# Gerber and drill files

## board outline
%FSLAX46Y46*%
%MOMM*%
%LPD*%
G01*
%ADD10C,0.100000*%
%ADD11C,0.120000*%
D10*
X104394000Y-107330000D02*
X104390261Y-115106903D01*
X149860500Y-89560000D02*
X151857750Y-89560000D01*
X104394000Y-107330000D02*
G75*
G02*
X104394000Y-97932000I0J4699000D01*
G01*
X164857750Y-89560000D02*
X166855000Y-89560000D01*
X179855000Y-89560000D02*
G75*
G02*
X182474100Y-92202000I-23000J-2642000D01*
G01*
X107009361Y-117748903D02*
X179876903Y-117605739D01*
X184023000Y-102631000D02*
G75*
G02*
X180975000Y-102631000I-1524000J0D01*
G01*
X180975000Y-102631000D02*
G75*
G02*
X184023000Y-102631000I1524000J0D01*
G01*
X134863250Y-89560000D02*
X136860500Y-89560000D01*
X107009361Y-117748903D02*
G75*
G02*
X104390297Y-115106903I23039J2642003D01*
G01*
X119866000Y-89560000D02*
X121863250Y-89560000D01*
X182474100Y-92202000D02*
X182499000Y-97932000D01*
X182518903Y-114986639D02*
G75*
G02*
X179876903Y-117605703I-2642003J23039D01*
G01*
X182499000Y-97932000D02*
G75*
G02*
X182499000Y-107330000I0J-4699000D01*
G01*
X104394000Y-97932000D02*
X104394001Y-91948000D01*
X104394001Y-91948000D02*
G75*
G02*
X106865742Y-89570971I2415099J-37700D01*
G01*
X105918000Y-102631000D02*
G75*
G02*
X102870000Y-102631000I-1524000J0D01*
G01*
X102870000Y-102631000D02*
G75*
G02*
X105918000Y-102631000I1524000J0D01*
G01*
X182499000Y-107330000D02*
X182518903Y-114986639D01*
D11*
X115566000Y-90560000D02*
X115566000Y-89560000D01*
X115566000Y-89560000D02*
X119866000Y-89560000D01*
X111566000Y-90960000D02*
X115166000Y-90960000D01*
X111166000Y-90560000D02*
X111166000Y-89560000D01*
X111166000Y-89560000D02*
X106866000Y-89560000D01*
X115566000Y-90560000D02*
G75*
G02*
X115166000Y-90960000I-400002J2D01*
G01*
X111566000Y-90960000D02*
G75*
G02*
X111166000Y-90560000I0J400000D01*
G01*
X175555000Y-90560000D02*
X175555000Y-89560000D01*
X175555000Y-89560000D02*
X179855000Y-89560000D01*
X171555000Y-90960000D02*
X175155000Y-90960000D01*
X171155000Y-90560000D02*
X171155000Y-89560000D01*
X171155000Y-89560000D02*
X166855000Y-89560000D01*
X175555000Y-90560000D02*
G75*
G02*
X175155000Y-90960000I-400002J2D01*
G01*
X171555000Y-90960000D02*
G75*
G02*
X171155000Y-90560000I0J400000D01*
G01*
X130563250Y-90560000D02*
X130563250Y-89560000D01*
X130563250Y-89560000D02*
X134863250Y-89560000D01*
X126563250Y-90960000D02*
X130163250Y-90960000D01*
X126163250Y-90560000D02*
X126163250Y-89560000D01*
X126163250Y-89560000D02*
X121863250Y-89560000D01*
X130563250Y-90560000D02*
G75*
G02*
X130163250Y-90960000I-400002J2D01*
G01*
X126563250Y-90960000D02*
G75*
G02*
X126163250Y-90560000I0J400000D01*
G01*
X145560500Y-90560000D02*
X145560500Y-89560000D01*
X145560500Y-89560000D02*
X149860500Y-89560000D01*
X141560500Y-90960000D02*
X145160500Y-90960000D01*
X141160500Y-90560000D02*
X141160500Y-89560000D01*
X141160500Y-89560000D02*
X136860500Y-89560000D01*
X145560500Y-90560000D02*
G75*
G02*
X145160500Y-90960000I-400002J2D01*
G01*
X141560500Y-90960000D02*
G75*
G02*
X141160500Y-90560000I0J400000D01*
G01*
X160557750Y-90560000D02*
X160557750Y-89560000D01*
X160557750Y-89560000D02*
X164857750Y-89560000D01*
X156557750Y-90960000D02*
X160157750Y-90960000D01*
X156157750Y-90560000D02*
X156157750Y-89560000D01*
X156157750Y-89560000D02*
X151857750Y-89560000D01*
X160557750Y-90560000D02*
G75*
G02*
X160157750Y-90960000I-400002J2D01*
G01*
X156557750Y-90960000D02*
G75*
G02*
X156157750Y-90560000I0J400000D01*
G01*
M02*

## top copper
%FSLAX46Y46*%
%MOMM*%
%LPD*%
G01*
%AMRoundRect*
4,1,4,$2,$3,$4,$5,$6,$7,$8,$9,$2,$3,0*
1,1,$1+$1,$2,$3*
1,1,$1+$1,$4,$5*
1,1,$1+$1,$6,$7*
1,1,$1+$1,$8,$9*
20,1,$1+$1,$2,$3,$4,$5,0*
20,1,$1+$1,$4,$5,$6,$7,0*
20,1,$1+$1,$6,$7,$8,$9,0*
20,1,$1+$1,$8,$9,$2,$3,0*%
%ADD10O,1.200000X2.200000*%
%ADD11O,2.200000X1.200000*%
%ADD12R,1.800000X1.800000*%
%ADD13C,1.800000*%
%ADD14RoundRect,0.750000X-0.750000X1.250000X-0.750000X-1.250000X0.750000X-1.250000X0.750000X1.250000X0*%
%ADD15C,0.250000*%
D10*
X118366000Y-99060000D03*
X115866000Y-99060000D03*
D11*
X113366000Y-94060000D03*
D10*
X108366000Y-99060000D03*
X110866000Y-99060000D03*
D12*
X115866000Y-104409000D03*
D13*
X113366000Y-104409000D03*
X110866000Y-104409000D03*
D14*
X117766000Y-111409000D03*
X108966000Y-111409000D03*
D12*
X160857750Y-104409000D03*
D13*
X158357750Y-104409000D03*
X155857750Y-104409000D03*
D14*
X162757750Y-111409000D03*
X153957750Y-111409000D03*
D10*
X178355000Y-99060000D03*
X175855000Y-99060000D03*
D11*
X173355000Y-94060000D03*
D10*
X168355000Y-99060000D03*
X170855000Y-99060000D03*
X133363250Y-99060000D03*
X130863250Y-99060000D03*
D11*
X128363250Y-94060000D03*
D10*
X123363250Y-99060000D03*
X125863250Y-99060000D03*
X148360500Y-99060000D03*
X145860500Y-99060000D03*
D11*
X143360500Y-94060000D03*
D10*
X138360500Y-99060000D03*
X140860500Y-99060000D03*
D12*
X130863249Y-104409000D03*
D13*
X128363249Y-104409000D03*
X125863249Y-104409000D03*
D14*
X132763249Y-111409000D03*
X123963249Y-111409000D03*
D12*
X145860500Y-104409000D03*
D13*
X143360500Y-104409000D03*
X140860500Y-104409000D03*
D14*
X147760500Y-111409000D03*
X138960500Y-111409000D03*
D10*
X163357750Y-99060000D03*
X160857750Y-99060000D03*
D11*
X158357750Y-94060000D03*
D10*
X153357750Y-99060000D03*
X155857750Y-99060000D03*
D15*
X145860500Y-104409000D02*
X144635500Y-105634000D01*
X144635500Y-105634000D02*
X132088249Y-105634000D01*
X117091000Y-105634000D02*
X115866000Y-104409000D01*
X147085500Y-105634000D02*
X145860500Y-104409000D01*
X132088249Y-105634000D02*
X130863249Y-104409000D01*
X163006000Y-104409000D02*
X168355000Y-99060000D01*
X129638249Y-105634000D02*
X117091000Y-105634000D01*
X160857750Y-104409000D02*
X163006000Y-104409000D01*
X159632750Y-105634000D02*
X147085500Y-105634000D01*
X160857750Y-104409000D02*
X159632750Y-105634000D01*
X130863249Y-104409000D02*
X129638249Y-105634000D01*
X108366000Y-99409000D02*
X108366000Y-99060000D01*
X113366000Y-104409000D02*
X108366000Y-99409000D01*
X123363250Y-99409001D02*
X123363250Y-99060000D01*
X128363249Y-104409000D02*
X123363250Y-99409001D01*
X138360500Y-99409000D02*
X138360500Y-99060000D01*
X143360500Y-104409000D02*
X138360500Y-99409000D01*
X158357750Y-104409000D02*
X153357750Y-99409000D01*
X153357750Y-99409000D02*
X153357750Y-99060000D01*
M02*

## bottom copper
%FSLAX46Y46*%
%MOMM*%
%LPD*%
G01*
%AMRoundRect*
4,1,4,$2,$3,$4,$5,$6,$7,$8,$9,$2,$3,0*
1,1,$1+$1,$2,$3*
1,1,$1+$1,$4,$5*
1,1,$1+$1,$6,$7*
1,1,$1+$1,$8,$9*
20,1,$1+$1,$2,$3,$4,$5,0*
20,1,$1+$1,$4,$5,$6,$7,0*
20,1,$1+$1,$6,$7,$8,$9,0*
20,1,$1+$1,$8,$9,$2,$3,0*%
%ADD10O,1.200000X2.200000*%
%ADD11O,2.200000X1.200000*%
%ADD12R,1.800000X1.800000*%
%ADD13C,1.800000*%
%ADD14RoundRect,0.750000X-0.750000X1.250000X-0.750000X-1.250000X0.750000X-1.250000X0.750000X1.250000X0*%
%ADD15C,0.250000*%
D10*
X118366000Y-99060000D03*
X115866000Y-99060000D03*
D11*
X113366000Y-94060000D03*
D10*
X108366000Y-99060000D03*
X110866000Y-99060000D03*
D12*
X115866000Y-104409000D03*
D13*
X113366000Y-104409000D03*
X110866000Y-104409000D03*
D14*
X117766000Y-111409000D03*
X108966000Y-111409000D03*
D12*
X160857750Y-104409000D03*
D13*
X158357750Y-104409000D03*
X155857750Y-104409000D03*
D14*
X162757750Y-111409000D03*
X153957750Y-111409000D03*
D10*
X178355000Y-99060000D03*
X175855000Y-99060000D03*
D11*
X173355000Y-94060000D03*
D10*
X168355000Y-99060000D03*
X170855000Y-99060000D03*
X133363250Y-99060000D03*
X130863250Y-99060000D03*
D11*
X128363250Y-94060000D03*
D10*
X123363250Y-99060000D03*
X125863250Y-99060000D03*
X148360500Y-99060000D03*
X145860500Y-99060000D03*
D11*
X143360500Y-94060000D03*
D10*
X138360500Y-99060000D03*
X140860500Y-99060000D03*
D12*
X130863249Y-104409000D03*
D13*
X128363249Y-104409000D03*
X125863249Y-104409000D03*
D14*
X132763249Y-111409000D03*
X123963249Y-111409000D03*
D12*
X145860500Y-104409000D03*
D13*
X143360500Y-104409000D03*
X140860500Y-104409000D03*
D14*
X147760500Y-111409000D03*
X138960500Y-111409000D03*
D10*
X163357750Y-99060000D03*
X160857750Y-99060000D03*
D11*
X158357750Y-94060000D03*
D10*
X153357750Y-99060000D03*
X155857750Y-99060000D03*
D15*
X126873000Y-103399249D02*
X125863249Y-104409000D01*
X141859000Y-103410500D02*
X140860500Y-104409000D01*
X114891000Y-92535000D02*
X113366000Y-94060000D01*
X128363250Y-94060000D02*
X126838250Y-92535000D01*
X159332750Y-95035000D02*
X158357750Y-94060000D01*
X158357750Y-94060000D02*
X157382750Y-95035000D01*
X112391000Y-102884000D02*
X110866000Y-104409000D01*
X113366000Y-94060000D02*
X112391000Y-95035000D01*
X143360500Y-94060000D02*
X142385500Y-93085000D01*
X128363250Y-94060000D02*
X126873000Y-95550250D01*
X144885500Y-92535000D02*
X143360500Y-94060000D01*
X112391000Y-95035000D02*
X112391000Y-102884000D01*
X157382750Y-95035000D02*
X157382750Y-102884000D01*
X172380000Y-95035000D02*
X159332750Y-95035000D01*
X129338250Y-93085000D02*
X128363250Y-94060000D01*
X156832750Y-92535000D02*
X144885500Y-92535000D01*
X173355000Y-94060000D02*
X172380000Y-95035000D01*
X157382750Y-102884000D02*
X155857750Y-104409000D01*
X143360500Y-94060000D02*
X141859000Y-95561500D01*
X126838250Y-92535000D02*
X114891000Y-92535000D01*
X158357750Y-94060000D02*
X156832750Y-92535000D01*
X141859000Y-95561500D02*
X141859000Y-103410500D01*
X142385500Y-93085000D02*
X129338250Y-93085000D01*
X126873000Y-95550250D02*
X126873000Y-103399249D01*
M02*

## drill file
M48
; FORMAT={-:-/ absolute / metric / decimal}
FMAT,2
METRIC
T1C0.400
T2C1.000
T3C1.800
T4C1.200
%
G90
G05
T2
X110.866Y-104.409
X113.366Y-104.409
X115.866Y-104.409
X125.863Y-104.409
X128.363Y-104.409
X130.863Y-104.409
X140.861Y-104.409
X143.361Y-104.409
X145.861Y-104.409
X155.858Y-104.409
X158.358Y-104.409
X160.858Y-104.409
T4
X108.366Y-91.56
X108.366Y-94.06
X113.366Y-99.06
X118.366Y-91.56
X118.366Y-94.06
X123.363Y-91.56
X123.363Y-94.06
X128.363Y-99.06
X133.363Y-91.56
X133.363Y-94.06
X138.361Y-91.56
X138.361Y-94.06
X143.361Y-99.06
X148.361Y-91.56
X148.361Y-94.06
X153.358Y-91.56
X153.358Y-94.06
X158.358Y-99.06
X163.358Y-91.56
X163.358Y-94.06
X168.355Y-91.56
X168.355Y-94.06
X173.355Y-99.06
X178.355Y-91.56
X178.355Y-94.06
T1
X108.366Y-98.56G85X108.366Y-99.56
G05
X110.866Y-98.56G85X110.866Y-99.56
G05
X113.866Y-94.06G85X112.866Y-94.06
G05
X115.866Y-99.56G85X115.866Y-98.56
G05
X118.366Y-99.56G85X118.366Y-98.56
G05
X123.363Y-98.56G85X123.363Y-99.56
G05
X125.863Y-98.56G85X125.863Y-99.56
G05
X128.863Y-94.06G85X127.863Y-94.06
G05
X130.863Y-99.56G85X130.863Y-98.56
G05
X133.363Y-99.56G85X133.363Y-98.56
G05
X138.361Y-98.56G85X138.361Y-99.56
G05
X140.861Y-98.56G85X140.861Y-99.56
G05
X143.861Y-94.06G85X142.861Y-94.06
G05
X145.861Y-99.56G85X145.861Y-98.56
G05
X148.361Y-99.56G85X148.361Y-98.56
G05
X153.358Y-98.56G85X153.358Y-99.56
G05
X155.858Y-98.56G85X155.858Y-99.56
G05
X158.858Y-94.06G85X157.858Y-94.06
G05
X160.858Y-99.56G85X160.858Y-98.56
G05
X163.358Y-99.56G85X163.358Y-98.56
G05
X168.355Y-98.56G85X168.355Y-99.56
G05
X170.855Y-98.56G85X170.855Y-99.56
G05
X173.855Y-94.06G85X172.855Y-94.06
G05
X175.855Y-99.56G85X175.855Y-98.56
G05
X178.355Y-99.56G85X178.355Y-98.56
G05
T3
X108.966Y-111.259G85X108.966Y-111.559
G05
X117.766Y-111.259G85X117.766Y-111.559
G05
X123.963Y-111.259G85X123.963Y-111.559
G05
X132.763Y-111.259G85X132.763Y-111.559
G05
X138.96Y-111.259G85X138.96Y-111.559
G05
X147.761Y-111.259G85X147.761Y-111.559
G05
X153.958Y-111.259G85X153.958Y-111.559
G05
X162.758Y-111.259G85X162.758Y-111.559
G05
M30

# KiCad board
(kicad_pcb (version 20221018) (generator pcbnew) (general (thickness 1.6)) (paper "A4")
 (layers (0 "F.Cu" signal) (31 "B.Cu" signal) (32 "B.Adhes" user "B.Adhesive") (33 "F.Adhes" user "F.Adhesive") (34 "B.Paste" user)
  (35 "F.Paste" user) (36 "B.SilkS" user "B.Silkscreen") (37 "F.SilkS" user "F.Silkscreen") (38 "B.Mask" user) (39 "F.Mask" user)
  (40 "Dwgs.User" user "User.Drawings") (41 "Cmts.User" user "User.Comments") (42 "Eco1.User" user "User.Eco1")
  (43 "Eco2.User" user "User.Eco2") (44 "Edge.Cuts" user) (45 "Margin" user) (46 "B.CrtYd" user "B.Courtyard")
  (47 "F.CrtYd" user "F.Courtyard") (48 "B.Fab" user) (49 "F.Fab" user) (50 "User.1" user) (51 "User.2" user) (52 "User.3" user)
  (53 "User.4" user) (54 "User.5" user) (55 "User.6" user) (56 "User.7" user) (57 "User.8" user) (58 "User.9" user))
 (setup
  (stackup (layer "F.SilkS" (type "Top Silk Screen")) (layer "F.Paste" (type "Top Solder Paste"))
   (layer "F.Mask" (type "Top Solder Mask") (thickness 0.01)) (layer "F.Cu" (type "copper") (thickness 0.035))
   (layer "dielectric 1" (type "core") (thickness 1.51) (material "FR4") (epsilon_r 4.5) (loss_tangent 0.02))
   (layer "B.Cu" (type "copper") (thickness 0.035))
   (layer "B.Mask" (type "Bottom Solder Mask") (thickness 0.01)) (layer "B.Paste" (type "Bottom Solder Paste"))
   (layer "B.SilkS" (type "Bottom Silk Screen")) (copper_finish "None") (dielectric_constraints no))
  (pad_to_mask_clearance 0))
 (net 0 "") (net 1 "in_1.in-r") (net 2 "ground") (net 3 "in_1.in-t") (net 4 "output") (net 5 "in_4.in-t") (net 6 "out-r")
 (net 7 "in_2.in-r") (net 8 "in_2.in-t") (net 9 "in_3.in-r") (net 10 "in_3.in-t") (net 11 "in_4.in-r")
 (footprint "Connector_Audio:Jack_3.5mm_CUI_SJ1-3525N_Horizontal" (layer "F.Cu") (at 113.366 94.06 180)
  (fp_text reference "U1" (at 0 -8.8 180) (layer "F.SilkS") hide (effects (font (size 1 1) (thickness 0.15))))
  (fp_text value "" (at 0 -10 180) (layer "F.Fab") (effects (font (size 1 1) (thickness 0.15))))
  (fp_line (start -2.2 3.5) (end -2.2 4.5) (stroke (width 0.12) (type solid)) (layer "Edge.Cuts"))
  (fp_line (start -2.2 4.5) (end -6.5 4.5) (stroke (width 0.12) (type solid)) (layer "Edge.Cuts"))
  (fp_line (start 1.8 3.1) (end -1.8 3.1) (stroke (width 0.12) (type solid)) (layer "Edge.Cuts"))
  (fp_line (start 2.2 3.5) (end 2.2 4.5) (stroke (width 0.12) (type solid)) (layer "Edge.Cuts"))
  (fp_line (start 2.2 4.5) (end 6.5 4.5) (stroke (width 0.12) (type solid)) (layer "Edge.Cuts"))
  (fp_arc (start -2.2 3.5) (mid -2.082842 3.217158) (end -1.8 3.1) (stroke (width 0.12) (type solid)) (layer "Edge.Cuts"))
  (fp_arc (start 1.8 3.1) (mid 2.082843 3.217157) (end 2.2 3.5) (stroke (width 0.12) (type solid)) (layer "Edge.Cuts"))
  (pad "" np_thru_hole circle (at -5 0 180) (size 1.2 1.2) (drill 1.2) (layers "*.Cu"))
  (pad "" np_thru_hole circle (at -5 2.5 180) (size 1.2 1.2) (drill 1.2) (layers "*.Cu"))
  (pad "" np_thru_hole circle (at 0 -5 180) (size 1.2 1.2) (drill 1.2) (layers "*.Cu"))
  (pad "" np_thru_hole circle (at 5 0 180) (size 1.2 1.2) (drill 1.2) (layers "*.Cu"))
  (pad "" np_thru_hole circle (at 5 2.5 180) (size 1.2 1.2) (drill 1.2) (layers "*.Cu"))
  (pad "R" thru_hole oval (at -5 -5 180) (size 1.2 2.2) (drill oval 0.4 1.4) (layers "*.Cu" "*.Mask") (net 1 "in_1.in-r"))
  (pad "RN" thru_hole oval (at -2.5 -5 180) (size 1.2 2.2) (drill oval 0.4 1.4) (layers "*.Cu" "*.Mask"))
  (pad "S" thru_hole oval (at 0 0 180) (size 2.2 1.2) (drill oval 1.4 0.4) (layers "*.Cu" "*.Mask") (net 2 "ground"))
  (pad "T" thru_hole oval (at 5 -5) (size 1.2 2.2) (drill oval 0.4 1.4) (layers "*.Cu" "*.Mask") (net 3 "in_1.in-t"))
  (pad "TN" thru_hole oval (at 2.5 -5) (size 1.2 2.2) (drill oval 0.4 1.4) (layers "*.Cu" "*.Mask")))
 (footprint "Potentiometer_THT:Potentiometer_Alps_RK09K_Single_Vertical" (layer "F.Cu") (at 115.866 104.409 -90)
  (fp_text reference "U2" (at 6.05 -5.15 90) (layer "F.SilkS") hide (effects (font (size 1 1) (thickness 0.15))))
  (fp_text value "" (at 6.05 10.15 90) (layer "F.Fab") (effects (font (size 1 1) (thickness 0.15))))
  (pad "1" thru_hole rect (at 0 0 270) (size 1.8 1.8) (drill 1) (layers "*.Cu" "*.Mask") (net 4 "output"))
  (pad "2" thru_hole circle (at 0 2.5 270) (size 1.8 1.8) (drill 1) (layers "*.Cu" "*.Mask") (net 3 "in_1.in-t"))
  (pad "3" thru_hole circle (at 0 5 270) (size 1.8 1.8) (drill 1) (layers "*.Cu" "*.Mask") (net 2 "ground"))
  (pad "MP" thru_hole roundrect (at 7 -1.9 270) (size 4 3) (drill oval 2.1 1.8) (layers "*.Cu" "*.Mask") (roundrect_rratio 0.25))
  (pad "MP" thru_hole roundrect (at 7 6.9 270) (size 4 3) (drill oval 2.1 1.8) (layers "*.Cu" "*.Mask") (roundrect_rratio 0.25)))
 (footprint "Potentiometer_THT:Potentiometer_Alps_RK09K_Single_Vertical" (layer "F.Cu") (at 160.85775 104.409 -90)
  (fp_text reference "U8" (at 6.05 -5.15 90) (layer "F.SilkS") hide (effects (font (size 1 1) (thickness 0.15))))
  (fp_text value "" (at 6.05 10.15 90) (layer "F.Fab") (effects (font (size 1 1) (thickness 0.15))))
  (pad "1" thru_hole rect (at 0 0 270) (size 1.8 1.8) (drill 1) (layers "*.Cu" "*.Mask") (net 4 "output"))
  (pad "2" thru_hole circle (at 0 2.5 270) (size 1.8 1.8) (drill 1) (layers "*.Cu" "*.Mask") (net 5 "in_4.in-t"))
  (pad "3" thru_hole circle (at 0 5 270) (size 1.8 1.8) (drill 1) (layers "*.Cu" "*.Mask") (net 2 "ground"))
  (pad "MP" thru_hole roundrect (at 7 -1.9 270) (size 4 3) (drill oval 2.1 1.8) (layers "*.Cu" "*.Mask") (roundrect_rratio 0.25))
  (pad "MP" thru_hole roundrect (at 7 6.9 270) (size 4 3) (drill oval 2.1 1.8) (layers "*.Cu" "*.Mask") (roundrect_rratio 0.25)))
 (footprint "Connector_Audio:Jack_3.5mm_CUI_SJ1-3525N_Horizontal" (layer "F.Cu") (at 173.355 94.06 180)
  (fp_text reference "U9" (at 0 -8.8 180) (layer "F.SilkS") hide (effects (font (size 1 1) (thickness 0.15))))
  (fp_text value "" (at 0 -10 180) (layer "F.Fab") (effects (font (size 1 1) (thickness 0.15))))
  (fp_line (start -2.2 3.5) (end -2.2 4.5) (stroke (width 0.12) (type solid)) (layer "Edge.Cuts"))
  (fp_line (start -2.2 4.5) (end -6.5 4.5) (stroke (width 0.12) (type solid)) (layer "Edge.Cuts"))
  (fp_line (start 1.8 3.1) (end -1.8 3.1) (stroke (width 0.12) (type solid)) (layer "Edge.Cuts"))
  (fp_line (start 2.2 3.5) (end 2.2 4.5) (stroke (width 0.12) (type solid)) (layer "Edge.Cuts"))
  (fp_line (start 2.2 4.5) (end 6.5 4.5) (stroke (width 0.12) (type solid)) (layer "Edge.Cuts"))
  (fp_arc (start -2.2 3.5) (mid -2.082842 3.217158) (end -1.8 3.1) (stroke (width 0.12) (type solid)) (layer "Edge.Cuts"))
  (fp_arc (start 1.8 3.1) (mid 2.082843 3.217157) (end 2.2 3.5) (stroke (width 0.12) (type solid)) (layer "Edge.Cuts"))
  (pad "" np_thru_hole circle (at -5 0 180) (size 1.2 1.2) (drill 1.2) (layers "*.Cu"))
  (pad "" np_thru_hole circle (at -5 2.5 180) (size 1.2 1.2) (drill 1.2) (layers "*.Cu"))
  (pad "" np_thru_hole circle (at 0 -5 180) (size 1.2 1.2) (drill 1.2) (layers "*.Cu"))
  (pad "" np_thru_hole circle (at 5 0 180) (size 1.2 1.2) (drill 1.2) (layers "*.Cu"))
  (pad "" np_thru_hole circle (at 5 2.5 180) (size 1.2 1.2) (drill 1.2) (layers "*.Cu"))
  (pad "R" thru_hole oval (at -5 -5 180) (size 1.2 2.2) (drill oval 0.4 1.4) (layers "*.Cu" "*.Mask") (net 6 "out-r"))
  (pad "RN" thru_hole oval (at -2.5 -5 180) (size 1.2 2.2) (drill oval 0.4 1.4) (layers "*.Cu" "*.Mask"))
  (pad "S" thru_hole oval (at 0 0 180) (size 2.2 1.2) (drill oval 1.4 0.4) (layers "*.Cu" "*.Mask") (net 2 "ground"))
  (pad "T" thru_hole oval (at 5 -5) (size 1.2 2.2) (drill oval 0.4 1.4) (layers "*.Cu" "*.Mask") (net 4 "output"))
  (pad "TN" thru_hole oval (at 2.5 -5) (size 1.2 2.2) (drill oval 0.4 1.4) (layers "*.Cu" "*.Mask")))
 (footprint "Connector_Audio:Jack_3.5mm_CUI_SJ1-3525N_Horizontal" (layer "F.Cu") (at 128.36325 94.06 180)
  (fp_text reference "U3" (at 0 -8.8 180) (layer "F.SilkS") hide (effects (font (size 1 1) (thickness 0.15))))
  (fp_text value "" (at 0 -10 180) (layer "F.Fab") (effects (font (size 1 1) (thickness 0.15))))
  (fp_line (start -2.2 3.5) (end -2.2 4.5) (stroke (width 0.12) (type solid)) (layer "Edge.Cuts"))
  (fp_line (start -2.2 4.5) (end -6.5 4.5) (stroke (width 0.12) (type solid)) (layer "Edge.Cuts"))
  (fp_line (start 1.8 3.1) (end -1.8 3.1) (stroke (width 0.12) (type solid)) (layer "Edge.Cuts"))
  (fp_line (start 2.2 3.5) (end 2.2 4.5) (stroke (width 0.12) (type solid)) (layer "Edge.Cuts"))
  (fp_line (start 2.2 4.5) (end 6.5 4.5) (stroke (width 0.12) (type solid)) (layer "Edge.Cuts"))
  (fp_arc (start -2.2 3.5) (mid -2.082842 3.217158) (end -1.8 3.1) (stroke (width 0.12) (type solid)) (layer "Edge.Cuts"))
  (fp_arc (start 1.8 3.1) (mid 2.082843 3.217157) (end 2.2 3.5) (stroke (width 0.12) (type solid)) (layer "Edge.Cuts"))
  (pad "" np_thru_hole circle (at -5 0 180) (size 1.2 1.2) (drill 1.2) (layers "*.Cu"))
  (pad "" np_thru_hole circle (at -5 2.5 180) (size 1.2 1.2) (drill 1.2) (layers "*.Cu"))
  (pad "" np_thru_hole circle (at 0 -5 180) (size 1.2 1.2) (drill 1.2) (layers "*.Cu"))
  (pad "" np_thru_hole circle (at 5 0 180) (size 1.2 1.2) (drill 1.2) (layers "*.Cu"))
  (pad "" np_thru_hole circle (at 5 2.5 180) (size 1.2 1.2) (drill 1.2) (layers "*.Cu"))
  (pad "R" thru_hole oval (at -5 -5 180) (size 1.2 2.2) (drill oval 0.4 1.4) (layers "*.Cu" "*.Mask") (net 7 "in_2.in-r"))
  (pad "RN" thru_hole oval (at -2.5 -5 180) (size 1.2 2.2) (drill oval 0.4 1.4) (layers "*.Cu" "*.Mask"))
  (pad "S" thru_hole oval (at 0 0 180) (size 2.2 1.2) (drill oval 1.4 0.4) (layers "*.Cu" "*.Mask") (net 2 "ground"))
  (pad "T" thru_hole oval (at 5 -5) (size 1.2 2.2) (drill oval 0.4 1.4) (layers "*.Cu" "*.Mask") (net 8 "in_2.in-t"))
  (pad "TN" thru_hole oval (at 2.5 -5) (size 1.2 2.2) (drill oval 0.4 1.4) (layers "*.Cu" "*.Mask")))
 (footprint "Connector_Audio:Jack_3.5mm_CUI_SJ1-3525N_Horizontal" (layer "F.Cu") (at 143.3605 94.06 180)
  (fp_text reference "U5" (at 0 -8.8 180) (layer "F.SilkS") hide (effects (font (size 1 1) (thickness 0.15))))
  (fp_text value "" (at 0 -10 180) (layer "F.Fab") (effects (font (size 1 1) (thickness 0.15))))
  (fp_line (start -2.2 3.5) (end -2.2 4.5) (stroke (width 0.12) (type solid)) (layer "Edge.Cuts"))
  (fp_line (start -2.2 4.5) (end -6.5 4.5) (stroke (width 0.12) (type solid)) (layer "Edge.Cuts"))
  (fp_line (start 1.8 3.1) (end -1.8 3.1) (stroke (width 0.12) (type solid)) (layer "Edge.Cuts"))
  (fp_line (start 2.2 3.5) (end 2.2 4.5) (stroke (width 0.12) (type solid)) (layer "Edge.Cuts"))
  (fp_line (start 2.2 4.5) (end 6.5 4.5) (stroke (width 0.12) (type solid)) (layer "Edge.Cuts"))
  (fp_arc (start -2.2 3.5) (mid -2.082842 3.217158) (end -1.8 3.1) (stroke (width 0.12) (type solid)) (layer "Edge.Cuts"))
  (fp_arc (start 1.8 3.1) (mid 2.082843 3.217157) (end 2.2 3.5) (stroke (width 0.12) (type solid)) (layer "Edge.Cuts"))
  (pad "" np_thru_hole circle (at -5 0 180) (size 1.2 1.2) (drill 1.2) (layers "*.Cu"))
  (pad "" np_thru_hole circle (at -5 2.5 180) (size 1.2 1.2) (drill 1.2) (layers "*.Cu"))
  (pad "" np_thru_hole circle (at 0 -5 180) (size 1.2 1.2) (drill 1.2) (layers "*.Cu"))
  (pad "" np_thru_hole circle (at 5 0 180) (size 1.2 1.2) (drill 1.2) (layers "*.Cu"))
  (pad "" np_thru_hole circle (at 5 2.5 180) (size 1.2 1.2) (drill 1.2) (layers "*.Cu"))
  (pad "R" thru_hole oval (at -5 -5 180) (size 1.2 2.2) (drill oval 0.4 1.4) (layers "*.Cu" "*.Mask") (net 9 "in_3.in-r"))
  (pad "RN" thru_hole oval (at -2.5 -5 180) (size 1.2 2.2) (drill oval 0.4 1.4) (layers "*.Cu" "*.Mask"))
  (pad "S" thru_hole oval (at 0 0 180) (size 2.2 1.2) (drill oval 1.4 0.4) (layers "*.Cu" "*.Mask") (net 2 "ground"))
  (pad "T" thru_hole oval (at 5 -5) (size 1.2 2.2) (drill oval 0.4 1.4) (layers "*.Cu" "*.Mask") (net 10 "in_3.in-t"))
  (pad "TN" thru_hole oval (at 2.5 -5) (size 1.2 2.2) (drill oval 0.4 1.4) (layers "*.Cu" "*.Mask")))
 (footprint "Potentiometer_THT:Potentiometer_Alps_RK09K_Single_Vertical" (layer "F.Cu") (at 130.863249 104.409 -90)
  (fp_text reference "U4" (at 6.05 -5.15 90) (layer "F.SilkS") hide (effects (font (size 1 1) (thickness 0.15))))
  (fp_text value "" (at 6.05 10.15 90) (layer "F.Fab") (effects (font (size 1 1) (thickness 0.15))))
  (pad "1" thru_hole rect (at 0 0 270) (size 1.8 1.8) (drill 1) (layers "*.Cu" "*.Mask") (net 4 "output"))
  (pad "2" thru_hole circle (at 0 2.5 270) (size 1.8 1.8) (drill 1) (layers "*.Cu" "*.Mask") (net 8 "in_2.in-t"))
  (pad "3" thru_hole circle (at 0 5 270) (size 1.8 1.8) (drill 1) (layers "*.Cu" "*.Mask") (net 2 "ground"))
  (pad "MP" thru_hole roundrect (at 7 -1.9 270) (size 4 3) (drill oval 2.1 1.8) (layers "*.Cu" "*.Mask") (roundrect_rratio 0.25))
  (pad "MP" thru_hole roundrect (at 7 6.9 270) (size 4 3) (drill oval 2.1 1.8) (layers "*.Cu" "*.Mask") (roundrect_rratio 0.25)))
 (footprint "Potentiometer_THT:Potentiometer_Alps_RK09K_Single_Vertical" (layer "F.Cu") (at 145.8605 104.409 -90)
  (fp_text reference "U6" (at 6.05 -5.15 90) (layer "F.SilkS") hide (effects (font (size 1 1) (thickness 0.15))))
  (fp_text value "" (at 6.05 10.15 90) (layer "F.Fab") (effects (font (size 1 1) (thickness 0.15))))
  (pad "1" thru_hole rect (at 0 0 270) (size 1.8 1.8) (drill 1) (layers "*.Cu" "*.Mask") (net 4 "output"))
  (pad "2" thru_hole circle (at 0 2.5 270) (size 1.8 1.8) (drill 1) (layers "*.Cu" "*.Mask") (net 10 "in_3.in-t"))
  (pad "3" thru_hole circle (at 0 5 270) (size 1.8 1.8) (drill 1) (layers "*.Cu" "*.Mask") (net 2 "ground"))
  (pad "MP" thru_hole roundrect (at 7 -1.9 270) (size 4 3) (drill oval 2.1 1.8) (layers "*.Cu" "*.Mask") (roundrect_rratio 0.25))
  (pad "MP" thru_hole roundrect (at 7 6.9 270) (size 4 3) (drill oval 2.1 1.8) (layers "*.Cu" "*.Mask") (roundrect_rratio 0.25)))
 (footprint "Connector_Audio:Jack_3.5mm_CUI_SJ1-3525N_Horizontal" (layer "F.Cu") (at 158.35775 94.06 180)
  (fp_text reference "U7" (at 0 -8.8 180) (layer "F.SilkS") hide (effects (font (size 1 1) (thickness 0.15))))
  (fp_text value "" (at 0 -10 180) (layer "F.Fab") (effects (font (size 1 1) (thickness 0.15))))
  (fp_line (start -2.2 3.5) (end -2.2 4.5) (stroke (width 0.12) (type solid)) (layer "Edge.Cuts"))
  (fp_line (start -2.2 4.5) (end -6.5 4.5) (stroke (width 0.12) (type solid)) (layer "Edge.Cuts"))
  (fp_line (start 1.8 3.1) (end -1.8 3.1) (stroke (width 0.12) (type solid)) (layer "Edge.Cuts"))
  (fp_line (start 2.2 3.5) (end 2.2 4.5) (stroke (width 0.12) (type solid)) (layer "Edge.Cuts"))
  (fp_line (start 2.2 4.5) (end 6.5 4.5) (stroke (width 0.12) (type solid)) (layer "Edge.Cuts"))
  (fp_arc (start -2.2 3.5) (mid -2.082842 3.217158) (end -1.8 3.1) (stroke (width 0.12) (type solid)) (layer "Edge.Cuts"))
  (fp_arc (start 1.8 3.1) (mid 2.082843 3.217157) (end 2.2 3.5) (stroke (width 0.12) (type solid)) (layer "Edge.Cuts"))
  (pad "" np_thru_hole circle (at -5 0 180) (size 1.2 1.2) (drill 1.2) (layers "*.Cu"))
  (pad "" np_thru_hole circle (at -5 2.5 180) (size 1.2 1.2) (drill 1.2) (layers "*.Cu"))
  (pad "" np_thru_hole circle (at 0 -5 180) (size 1.2 1.2) (drill 1.2) (layers "*.Cu"))
  (pad "" np_thru_hole circle (at 5 0 180) (size 1.2 1.2) (drill 1.2) (layers "*.Cu"))
  (pad "" np_thru_hole circle (at 5 2.5 180) (size 1.2 1.2) (drill 1.2) (layers "*.Cu"))
  (pad "R" thru_hole oval (at -5 -5 180) (size 1.2 2.2) (drill oval 0.4 1.4) (layers "*.Cu" "*.Mask") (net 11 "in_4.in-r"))
  (pad "RN" thru_hole oval (at -2.5 -5 180) (size 1.2 2.2) (drill oval 0.4 1.4) (layers "*.Cu" "*.Mask"))
  (pad "S" thru_hole oval (at 0 0 180) (size 2.2 1.2) (drill oval 1.4 0.4) (layers "*.Cu" "*.Mask") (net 2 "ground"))
  (pad "T" thru_hole oval (at 5 -5) (size 1.2 2.2) (drill oval 0.4 1.4) (layers "*.Cu" "*.Mask") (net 5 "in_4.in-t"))
  (pad "TN" thru_hole oval (at 2.5 -5) (size 1.2 2.2) (drill oval 0.4 1.4) (layers "*.Cu" "*.Mask")))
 (gr_line (start 104.394 107.33) (end 104.390261 115.106903) (stroke (width 0.1) (type default)) (layer "Edge.Cuts"))
 (gr_line (start 149.8605 89.56) (end 151.85775 89.56) (stroke (width 0.1) (type default)) (layer "Edge.Cuts"))
 (gr_arc (start 104.394 107.33) (mid 99.695 102.631) (end 104.394 97.932) (stroke (width 0.1) (type default)) (layer "Edge.Cuts"))
 (gr_line (start 164.85775 89.56) (end 166.855 89.56) (stroke (width 0.1) (type default)) (layer "Edge.Cuts"))
 (gr_arc (start 179.855 89.56) (mid 181.708361 90.341903) (end 182.4741 92.202) (stroke (width 0.1) (type default)) (layer "Edge.Cuts"))
 (gr_line (start 107.009361 117.748903) (end 179.876903 117.605739) (stroke (width 0.1) (type default)) (layer "Edge.Cuts"))
 (gr_circle (center 182.499 102.631) (end 184.023 102.631) (stroke (width 0.1) (type default)) (fill none) (layer "Edge.Cuts"))
 (gr_line (start 134.86325 89.56) (end 136.8605 89.56) (stroke (width 0.1) (type default)) (layer "Edge.Cuts"))
 (gr_arc (start 107.009361 117.748903) (mid 105.156 116.967) (end 104.390261 115.106903) (stroke (width 0.1) (type default))
  (layer "Edge.Cuts"))
 (gr_line (start 119.866 89.56) (end 121.86325 89.56) (stroke (width 0.1) (type default)) (layer "Edge.Cuts"))
 (gr_line (start 182.4741 92.202) (end 182.499 97.932) (stroke (width 0.1) (type default)) (layer "Edge.Cuts"))
 (gr_arc (start 182.518903 114.986639) (mid 181.737 116.84) (end 179.876903 117.605739) (stroke (width 0.1) (type default))
  (layer "Edge.Cuts"))
 (gr_arc (start 182.499 97.932) (mid 187.198 102.631) (end 182.499 107.33) (stroke (width 0.1) (type default)) (layer "Edge.Cuts"))
 (gr_line (start 104.394 97.932) (end 104.394001 91.948) (stroke (width 0.1) (type default)) (layer "Edge.Cuts"))
 (gr_arc (start 104.394001 91.948) (mid 105.134828 90.244708) (end 106.865743 89.570939) (stroke (width 0.1) (type default))
  (layer "Edge.Cuts"))
 (gr_circle (center 104.394 102.631) (end 105.918 102.631) (stroke (width 0.1) (type default)) (fill none) (layer "Edge.Cuts"))
 (gr_line (start 182.499 107.33) (end 182.518903 114.986639) (stroke (width 0.1) (type default)) (layer "Edge.Cuts"))
 (segment (start 145.8605 104.409) (end 144.6355 105.634) (width 0.25) (layer "F.Cu") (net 4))
 (segment (start 144.6355 105.634) (end 132.088249 105.634) (width 0.25) (layer "F.Cu") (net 4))
 (segment (start 117.091 105.634) (end 115.866 104.409) (width 0.25) (layer "F.Cu") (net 4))
 (segment (start 147.0855 105.634) (end 145.8605 104.409) (width 0.25) (layer "F.Cu") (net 4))
 (segment (start 132.088249 105.634) (end 130.863249 104.409) (width 0.25) (layer "F.Cu") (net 4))
 (segment (start 163.006 104.409) (end 168.355 99.06) (width 0.25) (layer "F.Cu") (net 4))
 (segment (start 129.638249 105.634) (end 117.091 105.634) (width 0.25) (layer "F.Cu") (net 4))
 (segment (start 160.85775 104.409) (end 163.006 104.409) (width 0.25) (layer "F.Cu") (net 4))
 (segment (start 159.63275 105.634) (end 147.0855 105.634) (width 0.25) (layer "F.Cu") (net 4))
 (segment (start 160.85775 104.409) (end 159.63275 105.634) (width 0.25) (layer "F.Cu") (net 4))
 (segment (start 130.863249 104.409) (end 129.638249 105.634) (width 0.25) (layer "F.Cu") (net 4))
 (segment (start 108.366 99.409) (end 108.366 99.06) (width 0.25) (layer "F.Cu") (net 3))
 (segment (start 113.366 104.409) (end 108.366 99.409) (width 0.25) (layer "F.Cu") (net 3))
 (segment (start 126.873 103.399249) (end 125.863249 104.409) (width 0.25) (layer "B.Cu") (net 2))
 (segment (start 141.859 103.4105) (end 140.8605 104.409) (width 0.25) (layer "B.Cu") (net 2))
 (segment (start 114.891 92.535) (end 113.366 94.06) (width 0.25) (layer "B.Cu") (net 2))
 (segment (start 128.36325 94.06) (end 126.83825 92.535) (width 0.25) (layer "B.Cu") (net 2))
 (segment (start 159.33275 95.035) (end 158.35775 94.06) (width 0.25) (layer "B.Cu") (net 2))
 (segment (start 158.35775 94.06) (end 157.38275 95.035) (width 0.25) (layer "B.Cu") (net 2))
 (segment (start 112.391 102.884) (end 110.866 104.409) (width 0.25) (layer "B.Cu") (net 2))
 (segment (start 113.366 94.06) (end 112.391 95.035) (width 0.25) (layer "B.Cu") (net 2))
 (segment (start 143.3605 94.06) (end 142.3855 93.085) (width 0.25) (layer "B.Cu") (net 2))
 (segment (start 128.36325 94.06) (end 126.873 95.55025) (width 0.25) (layer "B.Cu") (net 2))
 (segment (start 144.8855 92.535) (end 143.3605 94.06) (width 0.25) (layer "B.Cu") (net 2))
 (segment (start 112.391 95.035) (end 112.391 102.884) (width 0.25) (layer "B.Cu") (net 2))
 (segment (start 157.38275 95.035) (end 157.38275 102.884) (width 0.25) (layer "B.Cu") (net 2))
 (segment (start 172.38 95.035) (end 159.33275 95.035) (width 0.25) (layer "B.Cu") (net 2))
 (segment (start 129.33825 93.085) (end 128.36325 94.06) (width 0.25) (layer "B.Cu") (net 2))
 (segment (start 156.83275 92.535) (end 144.8855 92.535) (width 0.25) (layer "B.Cu") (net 2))
 (segment (start 173.355 94.06) (end 172.38 95.035) (width 0.25) (layer "B.Cu") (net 2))
 (segment (start 157.38275 102.884) (end 155.85775 104.409) (width 0.25) (layer "B.Cu") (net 2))
 (segment (start 143.3605 94.06) (end 141.859 95.5615) (width 0.25) (layer "B.Cu") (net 2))
 (segment (start 126.83825 92.535) (end 114.891 92.535) (width 0.25) (layer "B.Cu") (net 2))
 (segment (start 158.35775 94.06) (end 156.83275 92.535) (width 0.25) (layer "B.Cu") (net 2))
 (segment (start 141.859 95.5615) (end 141.859 103.4105) (width 0.25) (layer "B.Cu") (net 2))
 (segment (start 142.3855 93.085) (end 129.33825 93.085) (width 0.25) (layer "B.Cu") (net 2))
 (segment (start 126.873 95.55025) (end 126.873 103.399249) (width 0.25) (layer "B.Cu") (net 2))
 (segment (start 123.36325 99.409001) (end 123.36325 99.06) (width 0.25) (layer "F.Cu") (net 8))
 (segment (start 128.363249 104.409) (end 123.36325 99.409001) (width 0.25) (layer "F.Cu") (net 8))
 (segment (start 138.3605 99.409) (end 138.3605 99.06) (width 0.25) (layer "F.Cu") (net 10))
 (segment (start 143.3605 104.409) (end 138.3605 99.409) (width 0.25) (layer "F.Cu") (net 10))
 (segment (start 158.35775 104.409) (end 153.35775 99.409) (width 0.25) (layer "F.Cu") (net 5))
 (segment (start 153.35775 99.409) (end 153.35775 99.06) (width 0.25) (layer "F.Cu") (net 5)))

